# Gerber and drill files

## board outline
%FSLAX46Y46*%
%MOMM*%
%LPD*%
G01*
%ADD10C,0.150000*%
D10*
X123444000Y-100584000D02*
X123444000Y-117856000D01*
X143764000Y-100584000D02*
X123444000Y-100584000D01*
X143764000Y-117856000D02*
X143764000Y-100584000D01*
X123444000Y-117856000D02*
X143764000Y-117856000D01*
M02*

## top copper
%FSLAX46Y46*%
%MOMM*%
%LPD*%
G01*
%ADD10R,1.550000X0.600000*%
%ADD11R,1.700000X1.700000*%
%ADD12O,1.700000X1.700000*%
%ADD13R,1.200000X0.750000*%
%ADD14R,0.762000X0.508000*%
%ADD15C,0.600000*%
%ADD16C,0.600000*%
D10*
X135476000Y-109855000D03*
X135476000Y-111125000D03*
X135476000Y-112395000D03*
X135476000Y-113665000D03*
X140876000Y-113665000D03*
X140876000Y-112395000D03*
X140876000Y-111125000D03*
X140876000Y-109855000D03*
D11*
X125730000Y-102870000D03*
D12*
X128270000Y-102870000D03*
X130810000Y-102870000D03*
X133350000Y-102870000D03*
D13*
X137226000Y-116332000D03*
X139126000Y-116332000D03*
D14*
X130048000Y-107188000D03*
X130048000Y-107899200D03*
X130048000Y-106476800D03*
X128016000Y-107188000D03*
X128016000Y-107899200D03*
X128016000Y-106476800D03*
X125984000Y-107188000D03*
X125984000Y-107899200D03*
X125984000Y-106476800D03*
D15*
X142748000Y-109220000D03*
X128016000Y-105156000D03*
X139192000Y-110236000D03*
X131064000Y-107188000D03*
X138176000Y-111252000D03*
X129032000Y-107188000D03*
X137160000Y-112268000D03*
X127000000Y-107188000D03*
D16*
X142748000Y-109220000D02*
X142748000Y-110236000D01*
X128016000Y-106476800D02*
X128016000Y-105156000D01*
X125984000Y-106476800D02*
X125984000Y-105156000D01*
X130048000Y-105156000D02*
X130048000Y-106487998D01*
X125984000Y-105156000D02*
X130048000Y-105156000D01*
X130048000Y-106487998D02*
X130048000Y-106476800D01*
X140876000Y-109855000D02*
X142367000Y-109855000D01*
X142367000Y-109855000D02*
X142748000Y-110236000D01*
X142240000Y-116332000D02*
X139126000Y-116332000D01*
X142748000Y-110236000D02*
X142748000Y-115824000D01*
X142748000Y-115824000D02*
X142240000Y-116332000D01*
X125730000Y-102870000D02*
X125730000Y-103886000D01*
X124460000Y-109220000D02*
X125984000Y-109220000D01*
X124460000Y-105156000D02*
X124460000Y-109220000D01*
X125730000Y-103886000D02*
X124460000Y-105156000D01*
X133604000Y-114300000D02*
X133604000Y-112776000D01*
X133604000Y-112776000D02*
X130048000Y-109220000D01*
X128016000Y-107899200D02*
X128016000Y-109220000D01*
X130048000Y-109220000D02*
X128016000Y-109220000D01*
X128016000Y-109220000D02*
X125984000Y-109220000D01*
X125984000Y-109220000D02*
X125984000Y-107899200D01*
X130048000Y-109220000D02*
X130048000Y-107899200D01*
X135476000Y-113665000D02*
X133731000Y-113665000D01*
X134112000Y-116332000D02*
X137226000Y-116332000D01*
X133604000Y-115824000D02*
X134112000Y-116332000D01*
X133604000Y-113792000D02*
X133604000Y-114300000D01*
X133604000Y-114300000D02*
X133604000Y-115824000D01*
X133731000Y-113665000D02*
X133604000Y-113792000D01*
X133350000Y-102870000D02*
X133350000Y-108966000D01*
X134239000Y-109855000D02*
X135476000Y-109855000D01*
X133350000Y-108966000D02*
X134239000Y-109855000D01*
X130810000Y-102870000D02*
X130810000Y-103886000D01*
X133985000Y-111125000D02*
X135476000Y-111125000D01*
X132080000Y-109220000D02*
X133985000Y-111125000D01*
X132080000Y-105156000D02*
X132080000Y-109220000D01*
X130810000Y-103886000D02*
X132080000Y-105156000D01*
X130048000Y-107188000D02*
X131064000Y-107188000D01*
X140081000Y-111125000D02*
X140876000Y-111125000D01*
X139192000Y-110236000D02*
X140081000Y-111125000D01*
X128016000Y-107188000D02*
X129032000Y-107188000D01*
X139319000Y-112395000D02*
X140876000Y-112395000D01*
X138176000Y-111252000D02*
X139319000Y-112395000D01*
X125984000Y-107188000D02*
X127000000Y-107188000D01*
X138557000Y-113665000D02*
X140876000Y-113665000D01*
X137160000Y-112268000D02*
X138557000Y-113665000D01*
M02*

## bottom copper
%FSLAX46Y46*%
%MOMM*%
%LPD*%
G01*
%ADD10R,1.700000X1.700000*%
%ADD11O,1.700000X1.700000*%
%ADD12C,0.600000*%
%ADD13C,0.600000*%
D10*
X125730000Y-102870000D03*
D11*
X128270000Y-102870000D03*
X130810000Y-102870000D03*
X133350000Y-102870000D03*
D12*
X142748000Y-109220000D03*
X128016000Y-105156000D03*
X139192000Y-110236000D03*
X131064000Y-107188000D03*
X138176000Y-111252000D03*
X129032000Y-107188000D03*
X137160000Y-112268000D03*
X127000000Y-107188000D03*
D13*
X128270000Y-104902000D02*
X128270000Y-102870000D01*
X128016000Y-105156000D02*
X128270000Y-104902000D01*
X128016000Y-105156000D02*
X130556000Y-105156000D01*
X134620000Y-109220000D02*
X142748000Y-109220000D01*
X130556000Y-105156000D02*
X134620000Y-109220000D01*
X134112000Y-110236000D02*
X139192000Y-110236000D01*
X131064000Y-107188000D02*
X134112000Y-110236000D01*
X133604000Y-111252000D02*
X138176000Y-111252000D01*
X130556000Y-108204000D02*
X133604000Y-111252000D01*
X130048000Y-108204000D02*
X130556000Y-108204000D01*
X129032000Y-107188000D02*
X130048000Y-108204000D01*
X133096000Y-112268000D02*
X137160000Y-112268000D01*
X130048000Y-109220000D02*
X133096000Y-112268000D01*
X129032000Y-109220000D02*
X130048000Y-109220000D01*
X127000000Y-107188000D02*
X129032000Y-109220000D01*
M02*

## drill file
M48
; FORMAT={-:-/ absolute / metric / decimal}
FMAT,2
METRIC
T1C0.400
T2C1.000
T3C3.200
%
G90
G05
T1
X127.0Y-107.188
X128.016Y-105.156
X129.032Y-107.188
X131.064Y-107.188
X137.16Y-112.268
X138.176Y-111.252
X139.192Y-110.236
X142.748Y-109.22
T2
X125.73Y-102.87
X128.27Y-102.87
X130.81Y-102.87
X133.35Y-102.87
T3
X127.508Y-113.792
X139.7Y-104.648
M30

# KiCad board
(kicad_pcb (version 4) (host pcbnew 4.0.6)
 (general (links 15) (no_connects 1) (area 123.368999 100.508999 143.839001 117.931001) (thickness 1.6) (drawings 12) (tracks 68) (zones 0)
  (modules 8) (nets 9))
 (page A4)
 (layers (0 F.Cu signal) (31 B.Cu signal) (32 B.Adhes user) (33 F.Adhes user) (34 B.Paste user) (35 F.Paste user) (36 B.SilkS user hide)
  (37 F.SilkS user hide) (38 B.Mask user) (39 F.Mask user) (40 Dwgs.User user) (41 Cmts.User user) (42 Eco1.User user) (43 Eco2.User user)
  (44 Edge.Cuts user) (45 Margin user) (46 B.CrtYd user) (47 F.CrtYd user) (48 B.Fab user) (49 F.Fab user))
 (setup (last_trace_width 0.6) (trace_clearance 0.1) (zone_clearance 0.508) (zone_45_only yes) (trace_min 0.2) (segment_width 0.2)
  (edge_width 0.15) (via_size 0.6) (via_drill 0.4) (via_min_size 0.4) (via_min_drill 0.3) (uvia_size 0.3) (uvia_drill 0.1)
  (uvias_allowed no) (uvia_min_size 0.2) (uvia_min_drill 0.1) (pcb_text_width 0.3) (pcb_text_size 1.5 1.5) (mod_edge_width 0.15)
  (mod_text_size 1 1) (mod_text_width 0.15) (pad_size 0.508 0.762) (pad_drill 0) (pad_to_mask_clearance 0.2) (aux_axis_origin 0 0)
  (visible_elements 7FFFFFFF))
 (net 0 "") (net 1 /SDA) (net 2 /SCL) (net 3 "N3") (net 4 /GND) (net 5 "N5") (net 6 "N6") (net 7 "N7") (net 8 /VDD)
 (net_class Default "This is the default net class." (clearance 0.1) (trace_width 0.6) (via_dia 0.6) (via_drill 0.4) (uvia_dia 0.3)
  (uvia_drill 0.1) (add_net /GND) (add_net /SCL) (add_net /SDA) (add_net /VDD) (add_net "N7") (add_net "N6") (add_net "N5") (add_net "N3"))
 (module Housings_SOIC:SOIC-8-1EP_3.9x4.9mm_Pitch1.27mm (layer F.Cu) (at 138.176 111.76)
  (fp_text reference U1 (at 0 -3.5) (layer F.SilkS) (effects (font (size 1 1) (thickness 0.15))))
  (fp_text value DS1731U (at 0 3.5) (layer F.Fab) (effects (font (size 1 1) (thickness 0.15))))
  (pad 1 smd rect (at -2.7 -1.905) (size 1.55 0.6) (layers F.Cu F.Paste F.Mask) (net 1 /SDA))
  (pad 2 smd rect (at -2.7 -0.635) (size 1.55 0.6) (layers F.Cu F.Paste F.Mask) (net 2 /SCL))
  (pad 3 smd rect (at -2.7 0.635) (size 1.55 0.6) (layers F.Cu F.Paste F.Mask) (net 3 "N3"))
  (pad 4 smd rect (at -2.7 1.905) (size 1.55 0.6) (layers F.Cu F.Paste F.Mask) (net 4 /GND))
  (pad 5 smd rect (at 2.7 1.905) (size 1.55 0.6) (layers F.Cu F.Paste F.Mask) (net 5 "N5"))
  (pad 6 smd rect (at 2.7 0.635) (size 1.55 0.6) (layers F.Cu F.Paste F.Mask) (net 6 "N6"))
  (pad 7 smd rect (at 2.7 -0.635) (size 1.55 0.6) (layers F.Cu F.Paste F.Mask) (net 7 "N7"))
  (pad 8 smd rect (at 2.7 -1.905) (size 1.55 0.6) (layers F.Cu F.Paste F.Mask) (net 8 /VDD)))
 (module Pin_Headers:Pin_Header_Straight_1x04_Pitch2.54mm (layer F.Cu) (at 125.73 102.87 90)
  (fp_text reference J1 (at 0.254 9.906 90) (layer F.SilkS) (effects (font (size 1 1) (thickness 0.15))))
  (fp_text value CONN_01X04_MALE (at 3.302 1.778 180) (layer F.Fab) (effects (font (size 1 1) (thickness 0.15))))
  (pad 1 thru_hole rect (at 0 0 90) (size 1.7 1.7) (drill 1) (layers *.Cu *.Mask) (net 4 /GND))
  (pad 2 thru_hole oval (at 0 2.54 90) (size 1.7 1.7) (drill 1) (layers *.Cu *.Mask) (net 8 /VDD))
  (pad 3 thru_hole oval (at 0 5.08 90) (size 1.7 1.7) (drill 1) (layers *.Cu *.Mask) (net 2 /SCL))
  (pad 4 thru_hole oval (at 0 7.62 90) (size 1.7 1.7) (drill 1) (layers *.Cu *.Mask) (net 1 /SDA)))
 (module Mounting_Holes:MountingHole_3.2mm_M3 (layer F.Cu) (at 127.508 113.792)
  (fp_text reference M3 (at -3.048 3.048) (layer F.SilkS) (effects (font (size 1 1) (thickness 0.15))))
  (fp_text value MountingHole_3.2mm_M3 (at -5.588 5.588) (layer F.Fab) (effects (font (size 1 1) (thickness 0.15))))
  (pad 1 np_thru_hole circle (at 0 0) (size 3.2 3.2) (drill 3.2) (layers *.Cu *.Mask)))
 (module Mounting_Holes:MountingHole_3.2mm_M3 (layer F.Cu) (at 139.7 104.648)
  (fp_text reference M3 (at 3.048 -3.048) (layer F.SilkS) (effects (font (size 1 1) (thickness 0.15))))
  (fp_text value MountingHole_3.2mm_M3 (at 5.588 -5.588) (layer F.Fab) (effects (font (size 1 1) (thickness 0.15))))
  (pad 1 np_thru_hole circle (at 0 0) (size 3.2 3.2) (drill 3.2) (layers *.Cu *.Mask)))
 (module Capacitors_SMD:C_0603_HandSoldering (layer F.Cu) (at 138.176 116.332)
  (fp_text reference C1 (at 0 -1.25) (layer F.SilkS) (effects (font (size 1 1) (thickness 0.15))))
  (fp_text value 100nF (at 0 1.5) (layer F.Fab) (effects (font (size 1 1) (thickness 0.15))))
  (pad 1 smd rect (at -0.95 0) (size 1.2 0.75) (layers F.Cu F.Paste F.Mask) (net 4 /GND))
  (pad 2 smd rect (at 0.95 0) (size 1.2 0.75) (layers F.Cu F.Paste F.Mask) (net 8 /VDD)))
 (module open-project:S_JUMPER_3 (layer F.Cu) (at 130.048 107.188 90)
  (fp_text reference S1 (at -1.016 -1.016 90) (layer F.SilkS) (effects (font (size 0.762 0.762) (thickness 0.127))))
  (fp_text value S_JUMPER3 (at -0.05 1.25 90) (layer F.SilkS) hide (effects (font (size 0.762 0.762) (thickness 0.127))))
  (pad 2 smd rect (at 0 0 90) (size 0.508 0.762) (layers F.Cu F.Paste F.Mask) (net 7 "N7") (clearance 0.1))
  (pad 1 smd rect (at -0.7112 0 90) (size 0.508 0.762) (layers F.Cu F.Paste F.Mask) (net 4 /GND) (clearance 0.1))
  (pad 3 smd rect (at 0.7112 0 90) (size 0.508 0.762) (layers F.Cu F.Paste F.Mask) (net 8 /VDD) (clearance 0.1)))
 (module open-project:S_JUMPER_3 (layer F.Cu) (at 128.016 107.188 90)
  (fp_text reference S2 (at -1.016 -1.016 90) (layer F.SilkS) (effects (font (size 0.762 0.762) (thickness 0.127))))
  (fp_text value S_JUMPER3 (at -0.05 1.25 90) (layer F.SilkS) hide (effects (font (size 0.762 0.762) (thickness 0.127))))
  (pad 2 smd rect (at 0 0 90) (size 0.508 0.762) (layers F.Cu F.Paste F.Mask) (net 6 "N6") (clearance 0.1))
  (pad 1 smd rect (at -0.7112 0 90) (size 0.508 0.762) (layers F.Cu F.Paste F.Mask) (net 4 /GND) (clearance 0.1))
  (pad 3 smd rect (at 0.7112 0 90) (size 0.508 0.762) (layers F.Cu F.Paste F.Mask) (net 8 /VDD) (clearance 0.1)))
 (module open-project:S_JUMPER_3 (layer F.Cu) (at 125.984 107.188 90)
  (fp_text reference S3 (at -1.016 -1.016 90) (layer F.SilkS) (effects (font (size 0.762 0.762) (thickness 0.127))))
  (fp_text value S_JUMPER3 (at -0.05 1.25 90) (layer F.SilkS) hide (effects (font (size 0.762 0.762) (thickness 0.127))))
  (pad 2 smd rect (at 0 0 90) (size 0.508 0.762) (layers F.Cu F.Paste F.Mask) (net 5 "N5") (clearance 0.1))
  (pad 1 smd rect (at -0.7112 0 90) (size 0.508 0.762) (layers F.Cu F.Paste F.Mask) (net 4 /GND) (clearance 0.1))
  (pad 3 smd rect (at 0.7112 0 90) (size 0.508 0.762) (layers F.Cu F.Paste F.Mask) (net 8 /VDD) (clearance 0.1)))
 (gr_line (start 123.444 100.584) (end 123.444 117.856) (angle 90) (layer Edge.Cuts) (width 0.15))
 (gr_line (start 143.764 100.584) (end 123.444 100.584) (angle 90) (layer Edge.Cuts) (width 0.15))
 (gr_line (start 143.764 117.856) (end 143.764 100.584) (angle 90) (layer Edge.Cuts) (width 0.15))
 (gr_line (start 123.444 117.856) (end 143.764 117.856) (angle 90) (layer Edge.Cuts) (width 0.15))
 (segment (start 128.27 104.902) (end 128.27 102.87) (width 0.6) (layer B.Cu) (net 8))
 (segment (start 128.016 105.156) (end 128.27 104.902) (width 0.6) (layer B.Cu) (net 8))
 (segment (start 128.016 105.156) (end 130.556 105.156) (width 0.6) (layer B.Cu) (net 8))
 (segment (start 142.748 109.22) (end 142.748 110.236) (width 0.6) (layer F.Cu) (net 8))
 (via (at 142.748 109.22) (size 0.6) (drill 0.4) (layers F.Cu B.Cu) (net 8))
 (segment (start 134.62 109.22) (end 142.748 109.22) (width 0.6) (layer B.Cu) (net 8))
 (segment (start 130.556 105.156) (end 134.62 109.22) (width 0.6) (layer B.Cu) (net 8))
 (segment (start 128.016 106.4768) (end 128.016 105.156) (width 0.6) (layer F.Cu) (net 8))
 (via (at 128.016 105.156) (size 0.6) (drill 0.4) (layers F.Cu B.Cu) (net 8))
 (segment (start 125.984 106.4768) (end 125.984 105.156) (width 0.6) (layer F.Cu) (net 8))
 (segment (start 130.048 105.156) (end 130.048 106.487998) (width 0.6) (layer F.Cu) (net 8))
 (segment (start 125.984 105.156) (end 130.048 105.156) (width 0.6) (layer F.Cu) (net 8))
 (segment (start 130.048 106.487998) (end 130.048 106.4768) (width 0.6) (layer F.Cu) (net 8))
 (segment (start 140.876 109.855) (end 142.367 109.855) (width 0.6) (layer F.Cu) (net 8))
 (segment (start 142.367 109.855) (end 142.748 110.236) (width 0.6) (layer F.Cu) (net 8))
 (segment (start 142.24 116.332) (end 139.126 116.332) (width 0.6) (layer F.Cu) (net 8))
 (segment (start 142.748 110.236) (end 142.748 115.824) (width 0.6) (layer F.Cu) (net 8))
 (segment (start 142.748 115.824) (end 142.24 116.332) (width 0.6) (layer F.Cu) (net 8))
 (segment (start 125.73 102.87) (end 125.73 103.886) (width 0.6) (layer F.Cu) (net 4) (status 400000))
 (segment (start 124.46 109.22) (end 125.984 109.22) (width 0.6) (layer F.Cu) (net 4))
 (segment (start 124.46 105.156) (end 124.46 109.22) (width 0.6) (layer F.Cu) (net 4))
 (segment (start 125.73 103.886) (end 124.46 105.156) (width 0.6) (layer F.Cu) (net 4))
 (segment (start 133.604 114.3) (end 133.604 112.776) (width 0.6) (layer F.Cu) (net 4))
 (segment (start 133.604 112.776) (end 130.048 109.22) (width 0.6) (layer F.Cu) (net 4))
 (segment (start 128.016 107.8992) (end 128.016 109.22) (width 0.6) (layer F.Cu) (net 4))
 (segment (start 130.048 109.22) (end 128.016 109.22) (width 0.6) (layer F.Cu) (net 4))
 (segment (start 128.016 109.22) (end 125.984 109.22) (width 0.6) (layer F.Cu) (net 4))
 (segment (start 125.984 109.22) (end 125.984 107.8992) (width 0.6) (layer F.Cu) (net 4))
 (segment (start 130.048 109.22) (end 130.048 107.8992) (width 0.6) (layer F.Cu) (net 4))
 (segment (start 135.476 113.665) (end 133.731 113.665) (width 0.6) (layer F.Cu) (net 4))
 (segment (start 134.112 116.332) (end 137.226 116.332) (width 0.6) (layer F.Cu) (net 4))
 (segment (start 133.604 115.824) (end 134.112 116.332) (width 0.6) (layer F.Cu) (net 4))
 (segment (start 133.604 113.792) (end 133.604 114.3) (width 0.6) (layer F.Cu) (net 4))
 (segment (start 133.604 114.3) (end 133.604 115.824) (width 0.6) (layer F.Cu) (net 4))
 (segment (start 133.731 113.665) (end 133.604 113.792) (width 0.6) (layer F.Cu) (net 4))
 (segment (start 133.35 102.87) (end 133.35 108.966) (width 0.6) (layer F.Cu) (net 1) (status 400000))
 (segment (start 134.239 109.855) (end 135.476 109.855) (width 0.6) (layer F.Cu) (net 1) (status 800000))
 (segment (start 133.35 108.966) (end 134.239 109.855) (width 0.6) (layer F.Cu) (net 1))
 (segment (start 130.81 102.87) (end 130.81 103.886) (width 0.6) (layer F.Cu) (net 2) (status 400000))
 (segment (start 133.985 111.125) (end 135.476 111.125) (width 0.6) (layer F.Cu) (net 2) (status 800000))
 (segment (start 132.08 109.22) (end 133.985 111.125) (width 0.6) (layer F.Cu) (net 2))
 (segment (start 132.08 105.156) (end 132.08 109.22) (width 0.6) (layer F.Cu) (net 2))
 (segment (start 130.81 103.886) (end 132.08 105.156) (width 0.6) (layer F.Cu) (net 2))
 (segment (start 130.048 107.188) (end 131.064 107.188) (width 0.6) (layer F.Cu) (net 7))
 (segment (start 140.081 111.125) (end 140.876 111.125) (width 0.6) (layer F.Cu) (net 7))
 (segment (start 139.192 110.236) (end 140.081 111.125) (width 0.6) (layer F.Cu) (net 7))
 (via (at 139.192 110.236) (size 0.6) (drill 0.4) (layers F.Cu B.Cu) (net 7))
 (segment (start 134.112 110.236) (end 139.192 110.236) (width 0.6) (layer B.Cu) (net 7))
 (segment (start 131.064 107.188) (end 134.112 110.236) (width 0.6) (layer B.Cu) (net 7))
 (via (at 131.064 107.188) (size 0.6) (drill 0.4) (layers F.Cu B.Cu) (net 7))
 (segment (start 128.016 107.188) (end 129.032 107.188) (width 0.6) (layer F.Cu) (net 6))
 (segment (start 139.319 112.395) (end 140.876 112.395) (width 0.6) (layer F.Cu) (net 6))
 (segment (start 138.176 111.252) (end 139.319 112.395) (width 0.6) (layer F.Cu) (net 6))
 (via (at 138.176 111.252) (size 0.6) (drill 0.4) (layers F.Cu B.Cu) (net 6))
 (segment (start 133.604 111.252) (end 138.176 111.252) (width 0.6) (layer B.Cu) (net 6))
 (segment (start 130.556 108.204) (end 133.604 111.252) (width 0.6) (layer B.Cu) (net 6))
 (segment (start 130.048 108.204) (end 130.556 108.204) (width 0.6) (layer B.Cu) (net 6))
 (segment (start 129.032 107.188) (end 130.048 108.204) (width 0.6) (layer B.Cu) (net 6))
 (via (at 129.032 107.188) (size 0.6) (drill 0.4) (layers F.Cu B.Cu) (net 6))
 (segment (start 125.984 107.188) (end 127 107.188) (width 0.6) (layer F.Cu) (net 5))
 (segment (start 138.557 113.665) (end 140.876 113.665) (width 0.6) (layer F.Cu) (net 5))
 (segment (start 137.16 112.268) (end 138.557 113.665) (width 0.6) (layer F.Cu) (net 5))
 (via (at 137.16 112.268) (size 0.6) (drill 0.4) (layers F.Cu B.Cu) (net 5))
 (segment (start 133.096 112.268) (end 137.16 112.268) (width 0.6) (layer B.Cu) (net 5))
 (segment (start 130.048 109.22) (end 133.096 112.268) (width 0.6) (layer B.Cu) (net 5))
 (segment (start 129.032 109.22) (end 130.048 109.22) (width 0.6) (layer B.Cu) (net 5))
 (segment (start 127 107.188) (end 129.032 109.22) (width 0.6) (layer B.Cu) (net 5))
 (via (at 127 107.188) (size 0.6) (drill 0.4) (layers F.Cu B.Cu) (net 5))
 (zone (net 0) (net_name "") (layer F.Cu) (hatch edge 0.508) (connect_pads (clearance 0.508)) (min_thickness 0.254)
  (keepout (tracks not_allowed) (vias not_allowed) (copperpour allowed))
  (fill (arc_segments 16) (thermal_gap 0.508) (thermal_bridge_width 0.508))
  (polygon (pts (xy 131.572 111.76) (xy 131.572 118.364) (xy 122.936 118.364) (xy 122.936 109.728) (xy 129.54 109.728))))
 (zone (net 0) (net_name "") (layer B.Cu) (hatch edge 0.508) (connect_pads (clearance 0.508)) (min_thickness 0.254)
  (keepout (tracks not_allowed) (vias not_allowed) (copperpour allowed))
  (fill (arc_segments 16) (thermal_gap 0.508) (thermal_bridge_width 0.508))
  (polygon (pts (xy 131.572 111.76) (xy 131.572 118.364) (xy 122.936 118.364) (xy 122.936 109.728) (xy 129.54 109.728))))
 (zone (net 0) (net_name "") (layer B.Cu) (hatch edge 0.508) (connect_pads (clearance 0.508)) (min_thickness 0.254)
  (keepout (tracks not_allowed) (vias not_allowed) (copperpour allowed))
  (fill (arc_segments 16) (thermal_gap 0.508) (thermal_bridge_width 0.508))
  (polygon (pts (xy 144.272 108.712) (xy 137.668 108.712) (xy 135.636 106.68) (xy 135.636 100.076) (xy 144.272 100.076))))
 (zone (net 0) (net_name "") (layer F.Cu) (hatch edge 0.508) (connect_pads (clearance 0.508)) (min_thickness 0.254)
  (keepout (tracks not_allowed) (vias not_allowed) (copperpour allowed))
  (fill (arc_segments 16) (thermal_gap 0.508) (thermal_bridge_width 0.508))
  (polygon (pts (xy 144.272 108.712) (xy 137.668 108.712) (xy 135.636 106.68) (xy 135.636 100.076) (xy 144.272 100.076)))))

